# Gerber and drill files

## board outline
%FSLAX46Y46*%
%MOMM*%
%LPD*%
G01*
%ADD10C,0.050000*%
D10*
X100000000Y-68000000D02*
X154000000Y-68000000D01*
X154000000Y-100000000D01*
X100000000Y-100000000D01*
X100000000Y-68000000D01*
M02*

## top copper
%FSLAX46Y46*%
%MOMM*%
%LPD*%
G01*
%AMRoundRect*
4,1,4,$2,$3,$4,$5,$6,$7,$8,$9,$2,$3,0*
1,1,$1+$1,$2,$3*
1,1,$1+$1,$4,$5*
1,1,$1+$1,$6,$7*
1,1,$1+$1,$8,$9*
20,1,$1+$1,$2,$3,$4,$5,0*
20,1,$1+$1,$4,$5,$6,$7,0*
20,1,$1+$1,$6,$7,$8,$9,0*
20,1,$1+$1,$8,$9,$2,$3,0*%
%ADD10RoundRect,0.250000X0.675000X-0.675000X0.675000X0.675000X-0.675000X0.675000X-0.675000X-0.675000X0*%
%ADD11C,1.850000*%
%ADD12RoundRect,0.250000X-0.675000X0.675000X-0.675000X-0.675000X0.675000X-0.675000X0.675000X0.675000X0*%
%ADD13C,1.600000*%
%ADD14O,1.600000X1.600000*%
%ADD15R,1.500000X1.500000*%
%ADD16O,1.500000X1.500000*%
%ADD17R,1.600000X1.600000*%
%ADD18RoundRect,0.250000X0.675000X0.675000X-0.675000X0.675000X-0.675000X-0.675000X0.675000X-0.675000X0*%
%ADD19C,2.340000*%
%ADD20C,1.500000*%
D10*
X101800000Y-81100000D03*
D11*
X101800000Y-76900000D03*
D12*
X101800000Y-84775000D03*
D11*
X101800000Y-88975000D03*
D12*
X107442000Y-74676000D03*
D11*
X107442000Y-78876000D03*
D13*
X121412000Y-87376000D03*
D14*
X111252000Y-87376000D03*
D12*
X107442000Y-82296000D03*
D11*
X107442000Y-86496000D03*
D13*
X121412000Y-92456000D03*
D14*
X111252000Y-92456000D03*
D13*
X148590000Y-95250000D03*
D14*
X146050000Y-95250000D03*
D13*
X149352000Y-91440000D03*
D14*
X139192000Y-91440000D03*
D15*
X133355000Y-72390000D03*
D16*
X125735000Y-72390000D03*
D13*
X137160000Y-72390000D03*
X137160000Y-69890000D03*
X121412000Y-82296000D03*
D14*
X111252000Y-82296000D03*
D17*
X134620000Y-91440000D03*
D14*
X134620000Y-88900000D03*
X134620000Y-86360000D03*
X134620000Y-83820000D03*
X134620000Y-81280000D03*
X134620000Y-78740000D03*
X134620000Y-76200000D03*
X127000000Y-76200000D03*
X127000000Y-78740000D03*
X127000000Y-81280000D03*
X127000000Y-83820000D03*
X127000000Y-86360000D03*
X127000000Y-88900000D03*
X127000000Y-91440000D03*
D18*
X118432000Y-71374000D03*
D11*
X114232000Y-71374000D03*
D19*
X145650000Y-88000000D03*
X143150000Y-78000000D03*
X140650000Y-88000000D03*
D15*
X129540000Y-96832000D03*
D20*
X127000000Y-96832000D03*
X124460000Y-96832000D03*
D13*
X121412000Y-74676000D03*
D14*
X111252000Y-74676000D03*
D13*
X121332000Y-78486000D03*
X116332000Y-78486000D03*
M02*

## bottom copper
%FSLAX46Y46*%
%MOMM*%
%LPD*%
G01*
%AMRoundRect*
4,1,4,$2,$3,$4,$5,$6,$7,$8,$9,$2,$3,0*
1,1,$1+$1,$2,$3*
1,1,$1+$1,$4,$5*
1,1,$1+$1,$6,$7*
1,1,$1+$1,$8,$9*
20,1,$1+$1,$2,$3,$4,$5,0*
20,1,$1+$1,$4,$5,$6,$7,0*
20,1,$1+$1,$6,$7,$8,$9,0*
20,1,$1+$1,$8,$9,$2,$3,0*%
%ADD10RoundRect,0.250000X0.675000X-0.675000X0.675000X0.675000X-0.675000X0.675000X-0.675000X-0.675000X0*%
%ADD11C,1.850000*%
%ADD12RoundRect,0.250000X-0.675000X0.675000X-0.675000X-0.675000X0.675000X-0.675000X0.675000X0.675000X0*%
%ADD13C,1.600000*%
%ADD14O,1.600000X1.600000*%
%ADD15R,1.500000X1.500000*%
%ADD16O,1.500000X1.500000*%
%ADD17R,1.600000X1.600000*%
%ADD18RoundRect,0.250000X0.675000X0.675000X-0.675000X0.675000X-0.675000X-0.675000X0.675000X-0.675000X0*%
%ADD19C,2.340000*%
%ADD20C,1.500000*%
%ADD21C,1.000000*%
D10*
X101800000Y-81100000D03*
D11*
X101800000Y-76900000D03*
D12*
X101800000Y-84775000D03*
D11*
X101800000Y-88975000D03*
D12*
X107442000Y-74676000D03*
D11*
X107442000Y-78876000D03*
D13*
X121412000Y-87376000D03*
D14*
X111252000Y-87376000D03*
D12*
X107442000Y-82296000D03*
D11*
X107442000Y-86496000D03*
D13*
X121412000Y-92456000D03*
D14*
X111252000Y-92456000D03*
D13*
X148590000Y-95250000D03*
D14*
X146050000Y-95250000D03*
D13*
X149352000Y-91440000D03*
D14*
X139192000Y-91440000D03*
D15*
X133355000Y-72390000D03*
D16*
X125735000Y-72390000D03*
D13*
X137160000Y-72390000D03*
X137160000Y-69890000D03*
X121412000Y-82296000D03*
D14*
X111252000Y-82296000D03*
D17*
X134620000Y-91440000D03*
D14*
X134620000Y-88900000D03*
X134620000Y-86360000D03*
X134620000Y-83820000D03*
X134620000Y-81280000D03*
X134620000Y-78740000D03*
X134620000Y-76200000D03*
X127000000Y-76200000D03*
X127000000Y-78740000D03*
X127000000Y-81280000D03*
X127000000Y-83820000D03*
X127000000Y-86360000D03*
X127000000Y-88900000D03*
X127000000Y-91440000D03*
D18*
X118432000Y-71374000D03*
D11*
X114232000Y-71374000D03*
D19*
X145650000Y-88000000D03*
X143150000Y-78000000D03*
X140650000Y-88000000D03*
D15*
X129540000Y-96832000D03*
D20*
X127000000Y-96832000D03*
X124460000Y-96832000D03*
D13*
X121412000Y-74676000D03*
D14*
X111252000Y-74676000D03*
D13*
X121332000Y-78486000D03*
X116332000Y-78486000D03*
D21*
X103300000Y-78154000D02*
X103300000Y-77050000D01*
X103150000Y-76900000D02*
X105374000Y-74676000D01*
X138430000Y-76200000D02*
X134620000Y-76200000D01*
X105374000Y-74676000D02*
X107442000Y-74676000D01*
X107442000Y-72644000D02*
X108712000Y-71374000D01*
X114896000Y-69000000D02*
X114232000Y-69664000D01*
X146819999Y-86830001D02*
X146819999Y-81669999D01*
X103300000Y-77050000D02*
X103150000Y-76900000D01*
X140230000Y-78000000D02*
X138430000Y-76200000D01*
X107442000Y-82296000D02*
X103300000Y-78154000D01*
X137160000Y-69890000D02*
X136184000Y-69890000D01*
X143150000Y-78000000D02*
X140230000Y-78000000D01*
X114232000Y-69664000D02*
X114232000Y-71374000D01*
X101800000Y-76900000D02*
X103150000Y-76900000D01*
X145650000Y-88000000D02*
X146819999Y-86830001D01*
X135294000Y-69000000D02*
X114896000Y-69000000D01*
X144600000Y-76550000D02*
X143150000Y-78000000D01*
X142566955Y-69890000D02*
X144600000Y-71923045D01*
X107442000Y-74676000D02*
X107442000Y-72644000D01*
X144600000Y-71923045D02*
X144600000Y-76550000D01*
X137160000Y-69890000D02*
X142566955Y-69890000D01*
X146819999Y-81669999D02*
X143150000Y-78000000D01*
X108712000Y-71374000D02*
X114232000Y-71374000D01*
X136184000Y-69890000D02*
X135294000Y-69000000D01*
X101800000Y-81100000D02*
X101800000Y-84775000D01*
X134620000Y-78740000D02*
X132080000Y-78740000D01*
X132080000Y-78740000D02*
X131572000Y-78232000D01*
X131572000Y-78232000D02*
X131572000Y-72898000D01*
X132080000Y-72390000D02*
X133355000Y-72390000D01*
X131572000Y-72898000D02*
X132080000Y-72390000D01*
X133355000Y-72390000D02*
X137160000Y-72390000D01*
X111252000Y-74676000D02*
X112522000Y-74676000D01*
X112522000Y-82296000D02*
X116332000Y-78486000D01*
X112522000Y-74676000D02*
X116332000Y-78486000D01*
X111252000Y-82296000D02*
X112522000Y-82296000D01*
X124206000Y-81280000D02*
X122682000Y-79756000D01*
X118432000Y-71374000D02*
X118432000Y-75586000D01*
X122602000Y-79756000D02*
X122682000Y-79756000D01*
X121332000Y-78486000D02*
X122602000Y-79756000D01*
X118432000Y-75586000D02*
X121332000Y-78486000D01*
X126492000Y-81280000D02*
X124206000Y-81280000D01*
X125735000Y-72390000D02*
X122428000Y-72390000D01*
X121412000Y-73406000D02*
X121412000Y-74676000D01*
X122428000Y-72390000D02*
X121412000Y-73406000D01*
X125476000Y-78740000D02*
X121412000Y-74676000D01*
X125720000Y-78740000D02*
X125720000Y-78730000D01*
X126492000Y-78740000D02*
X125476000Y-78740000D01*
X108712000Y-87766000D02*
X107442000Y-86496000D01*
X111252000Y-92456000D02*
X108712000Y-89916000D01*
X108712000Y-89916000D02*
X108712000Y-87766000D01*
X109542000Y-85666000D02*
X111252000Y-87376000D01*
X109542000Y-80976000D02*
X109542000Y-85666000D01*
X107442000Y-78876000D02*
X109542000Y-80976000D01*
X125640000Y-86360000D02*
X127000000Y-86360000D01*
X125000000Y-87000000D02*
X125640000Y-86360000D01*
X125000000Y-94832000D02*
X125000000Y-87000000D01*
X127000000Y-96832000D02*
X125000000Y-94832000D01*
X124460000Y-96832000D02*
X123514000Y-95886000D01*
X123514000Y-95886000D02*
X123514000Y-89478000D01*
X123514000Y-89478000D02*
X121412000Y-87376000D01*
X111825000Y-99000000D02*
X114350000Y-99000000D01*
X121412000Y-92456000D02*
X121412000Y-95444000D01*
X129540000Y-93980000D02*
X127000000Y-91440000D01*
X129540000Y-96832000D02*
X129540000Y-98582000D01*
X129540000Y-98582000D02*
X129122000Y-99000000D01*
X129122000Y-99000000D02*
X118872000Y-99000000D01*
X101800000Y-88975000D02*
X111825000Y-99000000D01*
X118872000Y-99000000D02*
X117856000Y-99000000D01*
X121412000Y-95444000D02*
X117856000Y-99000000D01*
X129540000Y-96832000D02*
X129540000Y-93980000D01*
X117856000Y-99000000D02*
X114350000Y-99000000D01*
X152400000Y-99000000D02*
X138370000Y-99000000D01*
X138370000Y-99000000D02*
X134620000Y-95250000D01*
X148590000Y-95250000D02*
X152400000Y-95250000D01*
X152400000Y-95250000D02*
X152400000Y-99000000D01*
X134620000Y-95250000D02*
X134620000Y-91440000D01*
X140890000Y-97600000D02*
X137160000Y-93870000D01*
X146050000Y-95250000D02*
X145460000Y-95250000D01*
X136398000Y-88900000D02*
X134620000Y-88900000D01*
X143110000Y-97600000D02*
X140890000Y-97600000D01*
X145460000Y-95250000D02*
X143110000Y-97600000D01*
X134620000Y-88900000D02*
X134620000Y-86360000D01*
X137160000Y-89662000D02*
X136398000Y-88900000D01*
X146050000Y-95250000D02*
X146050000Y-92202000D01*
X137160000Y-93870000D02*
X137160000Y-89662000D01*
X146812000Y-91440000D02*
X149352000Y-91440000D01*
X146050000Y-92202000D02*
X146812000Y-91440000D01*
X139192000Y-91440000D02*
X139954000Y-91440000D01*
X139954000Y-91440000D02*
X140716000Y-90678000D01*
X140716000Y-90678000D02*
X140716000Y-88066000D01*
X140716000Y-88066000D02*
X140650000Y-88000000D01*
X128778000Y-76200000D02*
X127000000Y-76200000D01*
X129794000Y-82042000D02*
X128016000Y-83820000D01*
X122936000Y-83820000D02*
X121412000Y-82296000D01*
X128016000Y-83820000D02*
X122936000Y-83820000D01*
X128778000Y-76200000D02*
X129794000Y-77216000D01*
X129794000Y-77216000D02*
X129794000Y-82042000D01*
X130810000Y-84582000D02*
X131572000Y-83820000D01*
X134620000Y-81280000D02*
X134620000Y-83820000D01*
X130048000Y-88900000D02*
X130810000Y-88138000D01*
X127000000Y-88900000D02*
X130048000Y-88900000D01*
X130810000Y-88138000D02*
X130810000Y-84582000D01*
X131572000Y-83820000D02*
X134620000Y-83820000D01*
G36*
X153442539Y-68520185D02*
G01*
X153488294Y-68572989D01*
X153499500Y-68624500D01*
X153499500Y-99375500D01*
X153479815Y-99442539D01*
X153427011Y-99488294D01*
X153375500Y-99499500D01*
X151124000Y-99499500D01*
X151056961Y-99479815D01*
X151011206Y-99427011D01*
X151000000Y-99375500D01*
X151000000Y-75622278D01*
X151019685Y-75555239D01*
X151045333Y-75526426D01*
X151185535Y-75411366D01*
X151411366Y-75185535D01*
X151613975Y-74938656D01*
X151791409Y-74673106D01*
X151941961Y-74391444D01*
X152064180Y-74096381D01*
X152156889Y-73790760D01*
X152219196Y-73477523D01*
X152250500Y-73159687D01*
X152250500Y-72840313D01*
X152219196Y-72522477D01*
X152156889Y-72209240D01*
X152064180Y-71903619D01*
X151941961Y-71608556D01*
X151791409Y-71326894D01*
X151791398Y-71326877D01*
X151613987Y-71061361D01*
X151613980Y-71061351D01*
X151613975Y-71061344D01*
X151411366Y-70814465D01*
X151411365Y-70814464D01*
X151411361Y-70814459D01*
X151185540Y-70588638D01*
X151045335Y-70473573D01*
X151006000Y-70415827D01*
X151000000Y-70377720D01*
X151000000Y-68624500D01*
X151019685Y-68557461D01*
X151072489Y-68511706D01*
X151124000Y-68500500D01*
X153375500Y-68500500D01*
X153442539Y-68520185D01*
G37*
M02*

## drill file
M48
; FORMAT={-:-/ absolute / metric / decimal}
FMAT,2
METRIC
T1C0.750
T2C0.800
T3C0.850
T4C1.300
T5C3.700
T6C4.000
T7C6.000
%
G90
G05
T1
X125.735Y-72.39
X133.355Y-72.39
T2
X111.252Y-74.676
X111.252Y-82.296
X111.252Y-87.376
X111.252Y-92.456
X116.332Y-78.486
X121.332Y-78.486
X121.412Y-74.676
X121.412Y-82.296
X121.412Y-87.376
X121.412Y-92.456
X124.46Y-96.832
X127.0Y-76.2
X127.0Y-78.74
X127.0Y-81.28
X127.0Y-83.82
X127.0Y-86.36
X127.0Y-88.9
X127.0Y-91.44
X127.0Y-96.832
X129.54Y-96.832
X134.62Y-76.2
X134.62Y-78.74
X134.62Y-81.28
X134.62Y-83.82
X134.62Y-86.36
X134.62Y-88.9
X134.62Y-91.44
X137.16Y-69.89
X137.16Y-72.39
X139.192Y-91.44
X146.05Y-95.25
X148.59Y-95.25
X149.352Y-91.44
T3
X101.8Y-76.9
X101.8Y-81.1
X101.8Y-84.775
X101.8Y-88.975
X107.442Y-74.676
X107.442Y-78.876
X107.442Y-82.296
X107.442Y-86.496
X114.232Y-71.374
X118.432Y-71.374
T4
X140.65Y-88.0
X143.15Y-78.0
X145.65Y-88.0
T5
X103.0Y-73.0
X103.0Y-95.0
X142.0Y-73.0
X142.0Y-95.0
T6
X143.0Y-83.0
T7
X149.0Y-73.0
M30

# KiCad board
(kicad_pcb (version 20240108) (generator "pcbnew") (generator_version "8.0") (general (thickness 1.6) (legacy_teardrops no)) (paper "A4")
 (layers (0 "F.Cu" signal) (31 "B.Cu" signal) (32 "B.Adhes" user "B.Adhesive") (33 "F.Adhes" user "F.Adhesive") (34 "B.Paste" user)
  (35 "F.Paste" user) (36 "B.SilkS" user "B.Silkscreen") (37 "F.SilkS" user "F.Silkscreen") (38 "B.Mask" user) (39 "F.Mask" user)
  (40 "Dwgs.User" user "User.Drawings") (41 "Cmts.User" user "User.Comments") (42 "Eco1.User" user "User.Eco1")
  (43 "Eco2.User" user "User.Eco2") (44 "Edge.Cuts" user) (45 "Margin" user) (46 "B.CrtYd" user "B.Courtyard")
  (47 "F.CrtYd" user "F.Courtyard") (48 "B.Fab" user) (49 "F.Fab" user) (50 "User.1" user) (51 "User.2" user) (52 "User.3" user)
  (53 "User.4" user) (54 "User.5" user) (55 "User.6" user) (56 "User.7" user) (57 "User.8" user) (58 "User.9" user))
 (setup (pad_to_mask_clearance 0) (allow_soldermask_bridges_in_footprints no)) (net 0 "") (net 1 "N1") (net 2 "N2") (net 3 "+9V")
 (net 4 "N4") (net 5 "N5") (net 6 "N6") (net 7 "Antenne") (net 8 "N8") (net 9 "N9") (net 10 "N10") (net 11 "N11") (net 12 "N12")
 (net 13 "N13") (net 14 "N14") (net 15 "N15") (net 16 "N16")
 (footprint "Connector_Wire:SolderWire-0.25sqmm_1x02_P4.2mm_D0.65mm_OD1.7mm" (layer "F.Cu") (at 101.8 81.1 90)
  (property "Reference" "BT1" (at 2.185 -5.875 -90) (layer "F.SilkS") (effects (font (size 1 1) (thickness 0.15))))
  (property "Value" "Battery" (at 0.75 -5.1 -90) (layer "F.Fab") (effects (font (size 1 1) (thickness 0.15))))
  (pad "1" thru_hole roundrect (at 0 0 90) (size 1.85 1.85) (drill 0.85) (layers "*.Cu" "*.Mask") (remove_unused_layers no)
   (roundrect_rratio 0.135135) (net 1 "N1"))
  (pad "2" thru_hole circle (at 4.2 0 90) (size 1.85 1.85) (drill 0.85) (layers "*.Cu" "*.Mask") (remove_unused_layers no) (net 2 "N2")))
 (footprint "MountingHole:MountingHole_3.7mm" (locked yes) (layer "F.Cu") (at 142 95)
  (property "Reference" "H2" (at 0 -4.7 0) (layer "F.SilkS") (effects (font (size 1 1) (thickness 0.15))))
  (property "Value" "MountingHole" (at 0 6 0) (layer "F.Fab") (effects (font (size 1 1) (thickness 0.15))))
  (pad "" np_thru_hole circle (at 0 0) (size 3.7 3.7) (drill 3.7) (layers "*.Cu" "*.Mask")))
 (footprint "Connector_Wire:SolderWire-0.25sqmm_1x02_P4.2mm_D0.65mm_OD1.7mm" (layer "F.Cu") (at 101.8 84.775 -90)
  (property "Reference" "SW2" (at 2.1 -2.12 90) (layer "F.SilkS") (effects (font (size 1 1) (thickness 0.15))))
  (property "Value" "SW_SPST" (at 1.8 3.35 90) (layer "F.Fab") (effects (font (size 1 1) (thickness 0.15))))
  (pad "1" thru_hole roundrect (at 0 0 270) (size 1.85 1.85) (drill 0.85) (layers "*.Cu" "*.Mask") (remove_unused_layers no)
   (roundrect_rratio 0.135135) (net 1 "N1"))
  (pad "2" thru_hole circle (at 4.2 0 270) (size 1.85 1.85) (drill 0.85) (layers "*.Cu" "*.Mask") (remove_unused_layers no) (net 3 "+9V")))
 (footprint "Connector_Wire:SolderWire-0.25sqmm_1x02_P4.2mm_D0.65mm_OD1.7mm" (layer "F.Cu") (at 107.442 74.676 -90)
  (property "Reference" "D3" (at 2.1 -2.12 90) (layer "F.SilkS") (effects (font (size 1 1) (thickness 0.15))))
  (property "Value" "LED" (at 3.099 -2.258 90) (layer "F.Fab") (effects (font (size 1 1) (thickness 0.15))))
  (pad "1" thru_hole roundrect (at 0 0 270) (size 1.85 1.85) (drill 0.85) (layers "*.Cu" "*.Mask") (remove_unused_layers no)
   (roundrect_rratio 0.135135) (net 2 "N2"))
  (pad "2" thru_hole circle (at 4.2 0 270) (size 1.85 1.85) (drill 0.85) (layers "*.Cu" "*.Mask") (remove_unused_layers no) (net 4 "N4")))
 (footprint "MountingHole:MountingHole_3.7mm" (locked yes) (layer "F.Cu") (at 142 73)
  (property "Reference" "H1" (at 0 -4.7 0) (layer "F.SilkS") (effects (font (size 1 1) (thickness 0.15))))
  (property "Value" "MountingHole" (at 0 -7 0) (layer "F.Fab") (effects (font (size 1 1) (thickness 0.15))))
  (pad "" np_thru_hole circle (at 0 0) (size 3.7 3.7) (drill 3.7) (layers "*.Cu" "*.Mask")))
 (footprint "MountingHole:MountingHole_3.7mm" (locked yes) (layer "F.Cu") (at 103 73)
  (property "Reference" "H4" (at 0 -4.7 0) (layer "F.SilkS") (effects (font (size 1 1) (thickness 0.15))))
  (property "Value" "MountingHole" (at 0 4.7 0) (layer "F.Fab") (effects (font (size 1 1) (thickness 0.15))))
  (pad "" np_thru_hole circle (at 0 0) (size 3.7 3.7) (drill 3.7) (layers "*.Cu" "*.Mask")))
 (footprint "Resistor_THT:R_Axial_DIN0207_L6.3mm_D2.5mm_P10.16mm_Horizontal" (layer "F.Cu") (at 121.412 87.376 180)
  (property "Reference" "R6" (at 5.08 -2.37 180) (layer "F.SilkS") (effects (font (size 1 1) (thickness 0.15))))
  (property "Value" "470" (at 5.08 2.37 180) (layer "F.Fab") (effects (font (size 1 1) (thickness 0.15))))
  (pad "1" thru_hole circle (at 0 0 180) (size 1.6 1.6) (drill 0.8) (layers "*.Cu" "*.Mask") (remove_unused_layers no) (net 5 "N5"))
  (pad "2" thru_hole oval (at 10.16 0 180) (size 1.6 1.6) (drill 0.8) (layers "*.Cu" "*.Mask") (remove_unused_layers no) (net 4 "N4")))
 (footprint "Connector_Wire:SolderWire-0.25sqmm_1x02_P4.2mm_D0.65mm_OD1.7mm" (layer "F.Cu") (at 107.442 82.296 -90)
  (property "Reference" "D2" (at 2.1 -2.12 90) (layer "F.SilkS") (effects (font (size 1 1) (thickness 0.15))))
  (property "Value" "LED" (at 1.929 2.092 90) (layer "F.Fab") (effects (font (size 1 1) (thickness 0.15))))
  (pad "1" thru_hole roundrect (at 0 0 270) (size 1.85 1.85) (drill 0.85) (layers "*.Cu" "*.Mask") (remove_unused_layers no)
   (roundrect_rratio 0.135135) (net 2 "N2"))
  (pad "2" thru_hole circle (at 4.2 0 270) (size 1.85 1.85) (drill 0.85) (layers "*.Cu" "*.Mask") (remove_unused_layers no) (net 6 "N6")))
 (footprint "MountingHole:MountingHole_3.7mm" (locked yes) (layer "F.Cu") (at 103 95)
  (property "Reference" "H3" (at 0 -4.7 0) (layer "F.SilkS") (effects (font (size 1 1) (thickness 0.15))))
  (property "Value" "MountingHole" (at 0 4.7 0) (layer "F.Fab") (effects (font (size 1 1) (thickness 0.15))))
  (pad "" np_thru_hole circle (at 0 0) (size 3.7 3.7) (drill 3.7) (layers "*.Cu" "*.Mask")))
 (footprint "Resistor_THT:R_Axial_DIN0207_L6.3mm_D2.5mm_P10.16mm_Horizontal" (layer "F.Cu") (at 121.412 92.456 180)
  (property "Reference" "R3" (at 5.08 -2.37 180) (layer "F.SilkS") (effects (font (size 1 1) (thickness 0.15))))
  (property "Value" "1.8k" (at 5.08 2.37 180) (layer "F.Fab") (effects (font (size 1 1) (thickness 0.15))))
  (pad "1" thru_hole circle (at 0 0 180) (size 1.6 1.6) (drill 0.8) (layers "*.Cu" "*.Mask") (remove_unused_layers no) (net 3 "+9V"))
  (pad "2" thru_hole oval (at 10.16 0 180) (size 1.6 1.6) (drill 0.8) (layers "*.Cu" "*.Mask") (remove_unused_layers no) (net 6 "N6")))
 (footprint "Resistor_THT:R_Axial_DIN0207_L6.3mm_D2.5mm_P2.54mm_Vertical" (layer "F.Cu") (at 148.59 95.25 180)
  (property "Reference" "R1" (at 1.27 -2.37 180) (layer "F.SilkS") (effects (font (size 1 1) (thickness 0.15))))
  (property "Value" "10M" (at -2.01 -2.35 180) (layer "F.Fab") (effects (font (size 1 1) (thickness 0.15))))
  (pad "1" thru_hole circle (at 0 0 180) (size 1.6 1.6) (drill 0.8) (layers "*.Cu" "*.Mask") (remove_unused_layers no) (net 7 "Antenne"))
  (pad "2" thru_hole oval (at 2.54 0 180) (size 1.6 1.6) (drill 0.8) (layers "*.Cu" "*.Mask") (remove_unused_layers no) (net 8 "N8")))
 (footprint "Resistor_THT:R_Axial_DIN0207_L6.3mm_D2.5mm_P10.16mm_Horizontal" (layer "F.Cu") (at 149.352 91.44 180)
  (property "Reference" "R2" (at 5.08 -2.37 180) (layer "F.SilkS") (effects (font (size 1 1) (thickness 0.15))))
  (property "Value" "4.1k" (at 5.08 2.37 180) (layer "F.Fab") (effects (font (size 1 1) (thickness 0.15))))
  (pad "1" thru_hole circle (at 0 0 180) (size 1.6 1.6) (drill 0.8) (layers "*.Cu" "*.Mask") (remove_unused_layers no) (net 8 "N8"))
  (pad "2" thru_hole oval (at 10.16 0 180) (size 1.6 1.6) (drill 0.8) (layers "*.Cu" "*.Mask") (remove_unused_layers no) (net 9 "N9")))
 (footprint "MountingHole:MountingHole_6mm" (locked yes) (layer "F.Cu") (at 149 73)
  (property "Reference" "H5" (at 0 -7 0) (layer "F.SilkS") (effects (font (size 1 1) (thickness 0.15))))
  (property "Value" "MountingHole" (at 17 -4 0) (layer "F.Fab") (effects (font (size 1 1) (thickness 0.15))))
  (pad "" np_thru_hole circle (at 0 0) (size 6 6) (drill 6) (layers "*.Cu" "*.Mask")))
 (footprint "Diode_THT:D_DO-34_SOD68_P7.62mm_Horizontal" (layer "F.Cu") (at 133.355 72.39 180)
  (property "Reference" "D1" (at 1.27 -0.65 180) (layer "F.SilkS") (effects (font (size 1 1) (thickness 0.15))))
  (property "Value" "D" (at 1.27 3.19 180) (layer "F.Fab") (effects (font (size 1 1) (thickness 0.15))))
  (pad "1" thru_hole rect (at 0 0 180) (size 1.5 1.5) (drill 0.75) (layers "*.Cu" "*.Mask") (remove_unused_layers no) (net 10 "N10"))
  (pad "2" thru_hole oval (at 7.62 0 180) (size 1.5 1.5) (drill 0.75) (layers "*.Cu" "*.Mask") (remove_unused_layers no) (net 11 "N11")))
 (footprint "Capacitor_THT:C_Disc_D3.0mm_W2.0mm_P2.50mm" (layer "F.Cu") (at 137.16 72.39 90)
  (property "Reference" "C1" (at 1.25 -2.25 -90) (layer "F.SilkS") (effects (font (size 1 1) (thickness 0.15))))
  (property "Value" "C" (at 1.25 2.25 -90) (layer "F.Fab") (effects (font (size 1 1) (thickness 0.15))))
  (pad "1" thru_hole circle (at 0 0 90) (size 1.6 1.6) (drill 0.8) (layers "*.Cu" "*.Mask") (remove_unused_layers no) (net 10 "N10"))
  (pad "2" thru_hole circle (at 2.5 0 90) (size 1.6 1.6) (drill 0.8) (layers "*.Cu" "*.Mask") (remove_unused_layers no) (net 2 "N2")))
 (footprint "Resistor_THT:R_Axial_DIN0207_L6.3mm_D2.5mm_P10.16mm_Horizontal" (layer "F.Cu") (at 121.412 82.296 180)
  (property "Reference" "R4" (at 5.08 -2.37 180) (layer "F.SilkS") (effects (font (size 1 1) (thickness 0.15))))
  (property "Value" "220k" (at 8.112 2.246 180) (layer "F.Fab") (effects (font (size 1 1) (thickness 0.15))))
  (pad "1" thru_hole circle (at 0 0 180) (size 1.6 1.6) (drill 0.8) (layers "*.Cu" "*.Mask") (remove_unused_layers no) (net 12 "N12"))
  (pad "2" thru_hole oval (at 10.16 0 180) (size 1.6 1.6) (drill 0.8) (layers "*.Cu" "*.Mask") (remove_unused_layers no) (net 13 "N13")))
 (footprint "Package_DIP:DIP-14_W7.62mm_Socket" (layer "F.Cu") (at 134.62 91.44 180)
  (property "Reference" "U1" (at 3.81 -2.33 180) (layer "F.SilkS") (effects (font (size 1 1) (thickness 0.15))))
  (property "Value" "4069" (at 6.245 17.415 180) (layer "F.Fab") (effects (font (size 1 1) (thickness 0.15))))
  (pad "1" thru_hole rect (at 0 0 180) (size 1.6 1.6) (drill 0.8) (layers "*.Cu" "*.Mask") (remove_unused_layers no) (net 7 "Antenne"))
  (pad "2" thru_hole oval (at 0 2.54 180) (size 1.6 1.6) (drill 0.8) (layers "*.Cu" "*.Mask") (remove_unused_layers no) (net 8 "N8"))
  (pad "3" thru_hole oval (at 0 5.08 180) (size 1.6 1.6) (drill 0.8) (layers "*.Cu" "*.Mask") (remove_unused_layers no) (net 8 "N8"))
  (pad "4" thru_hole oval (at 0 7.62 180) (size 1.6 1.6) (drill 0.8) (layers "*.Cu" "*.Mask") (remove_unused_layers no) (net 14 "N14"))
  (pad "5" thru_hole oval (at 0 10.16 180) (size 1.6 1.6) (drill 0.8) (layers "*.Cu" "*.Mask") (remove_unused_layers no) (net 14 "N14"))
  (pad "6" thru_hole oval (at 0 12.7 180) (size 1.6 1.6) (drill 0.8) (layers "*.Cu" "*.Mask") (remove_unused_layers no) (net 10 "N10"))
  (pad "7" thru_hole oval (at 0 15.24 180) (size 1.6 1.6) (drill 0.8) (layers "*.Cu" "*.Mask") (remove_unused_layers no) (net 2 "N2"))
  (pad "8" thru_hole oval (at 7.62 15.24 180) (size 1.6 1.6) (drill 0.8) (layers "*.Cu" "*.Mask") (remove_unused_layers no) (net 12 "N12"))
  (pad "9" thru_hole oval (at 7.62 12.7 180) (size 1.6 1.6) (drill 0.8) (layers "*.Cu" "*.Mask") (remove_unused_layers no) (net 11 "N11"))
  (pad "10" thru_hole oval (at 7.62 10.16 180) (size 1.6 1.6) (drill 0.8) (layers "*.Cu" "*.Mask") (remove_unused_layers no) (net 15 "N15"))
  (pad "11" thru_hole oval (at 7.62 7.62 180) (size 1.6 1.6) (drill 0.8) (layers "*.Cu" "*.Mask") (remove_unused_layers no) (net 12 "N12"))
  (pad "12" thru_hole oval (at 7.62 5.08 180) (size 1.6 1.6) (drill 0.8) (layers "*.Cu" "*.Mask") (remove_unused_layers no) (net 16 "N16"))
  (pad "13" thru_hole oval (at 7.62 2.54 180) (size 1.6 1.6) (drill 0.8) (layers "*.Cu" "*.Mask") (remove_unused_layers no) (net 14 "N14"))
  (pad "14" thru_hole oval (at 7.62 0 180) (size 1.6 1.6) (drill 0.8) (layers "*.Cu" "*.Mask") (remove_unused_layers no) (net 3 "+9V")))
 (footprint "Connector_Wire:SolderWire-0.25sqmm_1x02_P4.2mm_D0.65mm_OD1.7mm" (layer "F.Cu") (at 118.432 71.374 180)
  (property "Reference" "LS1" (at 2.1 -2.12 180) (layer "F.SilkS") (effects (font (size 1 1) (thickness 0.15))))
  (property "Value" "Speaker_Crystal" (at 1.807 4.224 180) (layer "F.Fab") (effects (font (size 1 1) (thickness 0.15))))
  (pad "1" thru_hole roundrect (at 0 0 180) (size 1.85 1.85) (drill 0.85) (layers "*.Cu" "*.Mask") (remove_unused_layers no)
   (roundrect_rratio 0.135135) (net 15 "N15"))
  (pad "2" thru_hole circle (at 4.2 0 180) (size 1.85 1.85) (drill 0.85) (layers "*.Cu" "*.Mask") (remove_unused_layers no) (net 2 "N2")))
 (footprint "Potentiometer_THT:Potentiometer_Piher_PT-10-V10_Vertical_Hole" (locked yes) (layer "F.Cu") (at 145.65 88 90)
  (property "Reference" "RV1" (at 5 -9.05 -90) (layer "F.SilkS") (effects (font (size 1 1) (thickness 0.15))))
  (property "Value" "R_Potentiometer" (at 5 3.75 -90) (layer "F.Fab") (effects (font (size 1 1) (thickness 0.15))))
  (pad "" np_thru_hole circle (at 5 -2.65 90) (size 4 4) (drill 4) (layers "*.Cu" "*.Mask"))
  (pad "1" thru_hole circle (at 0 0 90) (size 2.34 2.34) (drill 1.3) (layers "*.Cu" "*.Mask") (remove_unused_layers no) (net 2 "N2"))
  (pad "2" thru_hole circle (at 10 -2.5 90) (size 2.34 2.34) (drill 1.3) (layers "*.Cu" "*.Mask") (remove_unused_layers no) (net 2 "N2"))
  (pad "3" thru_hole circle (at 0 -5 90) (size 2.34 2.34) (drill 1.3) (layers "*.Cu" "*.Mask") (remove_unused_layers no) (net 9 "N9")))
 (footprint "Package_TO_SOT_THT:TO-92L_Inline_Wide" (layer "F.Cu") (at 129.54 96.832 180)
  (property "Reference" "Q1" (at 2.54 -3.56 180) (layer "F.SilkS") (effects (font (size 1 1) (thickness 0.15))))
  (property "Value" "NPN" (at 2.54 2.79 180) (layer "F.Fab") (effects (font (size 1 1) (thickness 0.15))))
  (pad "1" thru_hole rect (at 0 0 180) (size 1.5 1.5) (drill 0.8) (layers "*.Cu" "*.Mask") (remove_unused_layers no) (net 3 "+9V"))
  (pad "2" thru_hole circle (at 2.54 0 180) (size 1.5 1.5) (drill 0.8) (layers "*.Cu" "*.Mask") (remove_unused_layers no) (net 16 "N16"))
  (pad "3" thru_hole circle (at 5.08 0 180) (size 1.5 1.5) (drill 0.8) (layers "*.Cu" "*.Mask") (remove_unused_layers no) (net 5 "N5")))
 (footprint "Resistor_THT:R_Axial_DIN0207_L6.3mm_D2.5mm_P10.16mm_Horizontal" (layer "F.Cu") (at 121.412 74.676 180)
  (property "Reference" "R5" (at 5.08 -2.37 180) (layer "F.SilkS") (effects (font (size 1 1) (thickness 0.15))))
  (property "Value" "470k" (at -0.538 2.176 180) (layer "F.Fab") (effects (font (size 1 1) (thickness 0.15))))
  (pad "1" thru_hole circle (at 0 0 180) (size 1.6 1.6) (drill 0.8) (layers "*.Cu" "*.Mask") (remove_unused_layers no) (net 11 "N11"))
  (pad "2" thru_hole oval (at 10.16 0 180) (size 1.6 1.6) (drill 0.8) (layers "*.Cu" "*.Mask") (remove_unused_layers no) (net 13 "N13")))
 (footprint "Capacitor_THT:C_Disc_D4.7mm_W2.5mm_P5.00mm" (layer "F.Cu") (at 121.332 78.486 180)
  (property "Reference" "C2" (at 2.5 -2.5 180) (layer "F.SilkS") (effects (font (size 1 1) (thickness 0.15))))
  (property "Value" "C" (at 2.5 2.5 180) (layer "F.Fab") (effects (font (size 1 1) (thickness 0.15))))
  (pad "1" thru_hole circle (at 0 0 180) (size 1.6 1.6) (drill 0.8) (layers "*.Cu" "*.Mask") (remove_unused_layers no) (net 15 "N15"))
  (pad "2" thru_hole circle (at 5 0 180) (size 1.6 1.6) (drill 0.8) (layers "*.Cu" "*.Mask") (remove_unused_layers no) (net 13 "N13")))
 (gr_rect (start 100 68) (end 154 100) (locked yes) (stroke (width 0.05) (type default)) (fill none) (layer "Edge.Cuts"))
 (segment (start 103.3 78.154) (end 103.3 77.05) (width 1) (layer "B.Cu") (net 2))
 (segment (start 103.15 76.9) (end 105.374 74.676) (width 1) (layer "B.Cu") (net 2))
 (segment (start 138.43 76.2) (end 134.62 76.2) (width 1) (layer "B.Cu") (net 2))
 (segment (start 105.374 74.676) (end 107.442 74.676) (width 1) (layer "B.Cu") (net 2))
 (segment (start 107.442 72.644) (end 108.712 71.374) (width 1) (layer "B.Cu") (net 2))
 (segment (start 114.896 69) (end 114.232 69.664) (width 1) (layer "B.Cu") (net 2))
 (segment (start 146.819999 86.830001) (end 146.819999 81.669999) (width 1) (layer "B.Cu") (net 2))
 (segment (start 103.3 77.05) (end 103.15 76.9) (width 1) (layer "B.Cu") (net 2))
 (segment (start 140.23 78) (end 138.43 76.2) (width 1) (layer "B.Cu") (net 2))
 (segment (start 107.442 82.296) (end 103.3 78.154) (width 1) (layer "B.Cu") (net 2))
 (segment (start 137.16 69.89) (end 136.184 69.89) (width 1) (layer "B.Cu") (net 2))
 (segment (start 143.15 78) (end 140.23 78) (width 1) (layer "B.Cu") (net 2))
 (segment (start 114.232 69.664) (end 114.232 71.374) (width 1) (layer "B.Cu") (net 2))
 (segment (start 101.8 76.9) (end 103.15 76.9) (width 1) (layer "B.Cu") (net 2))
 (segment (start 145.65 88) (end 146.819999 86.830001) (width 1) (layer "B.Cu") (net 2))
 (segment (start 135.294 69) (end 114.896 69) (width 1) (layer "B.Cu") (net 2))
 (segment (start 144.6 76.55) (end 143.15 78) (width 1) (layer "B.Cu") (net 2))
 (segment (start 142.566955 69.89) (end 144.6 71.923045) (width 1) (layer "B.Cu") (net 2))
 (segment (start 107.442 74.676) (end 107.442 72.644) (width 1) (layer "B.Cu") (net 2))
 (segment (start 144.6 71.923045) (end 144.6 76.55) (width 1) (layer "B.Cu") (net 2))
 (segment (start 137.16 69.89) (end 142.566955 69.89) (width 1) (layer "B.Cu") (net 2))
 (segment (start 146.819999 81.669999) (end 143.15 78) (width 1) (layer "B.Cu") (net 2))
 (segment (start 108.712 71.374) (end 114.232 71.374) (width 1) (layer "B.Cu") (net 2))
 (segment (start 136.184 69.89) (end 135.294 69) (width 1) (layer "B.Cu") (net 2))
 (segment (start 101.8 81.1) (end 101.8 84.775) (width 1) (layer "B.Cu") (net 1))
 (segment (start 134.62 78.74) (end 132.08 78.74) (width 1) (layer "B.Cu") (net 10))
 (segment (start 132.08 78.74) (end 131.572 78.232) (width 1) (layer "B.Cu") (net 10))
 (segment (start 131.572 78.232) (end 131.572 72.898) (width 1) (layer "B.Cu") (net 10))
 (segment (start 132.08 72.39) (end 133.355 72.39) (width 1) (layer "B.Cu") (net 10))
 (segment (start 131.572 72.898) (end 132.08 72.39) (width 1) (layer "B.Cu") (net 10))
 (segment (start 133.355 72.39) (end 137.16 72.39) (width 1) (layer "B.Cu") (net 10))
 (segment (start 111.252 74.676) (end 112.522 74.676) (width 1) (layer "B.Cu") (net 13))
 (segment (start 112.522 82.296) (end 116.332 78.486) (width 1) (layer "B.Cu") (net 13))
 (segment (start 112.522 74.676) (end 116.332 78.486) (width 1) (layer "B.Cu") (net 13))
 (segment (start 111.252 82.296) (end 112.522 82.296) (width 1) (layer "B.Cu") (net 13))
 (segment (start 124.206 81.28) (end 122.682 79.756) (width 1) (layer "B.Cu") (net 15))
 (segment (start 118.432 71.374) (end 118.432 75.586) (width 1) (layer "B.Cu") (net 15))
 (segment (start 122.602 79.756) (end 122.682 79.756) (width 1) (layer "B.Cu") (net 15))
 (segment (start 121.332 78.486) (end 122.602 79.756) (width 1) (layer "B.Cu") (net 15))
 (segment (start 118.432 75.586) (end 121.332 78.486) (width 1) (layer "B.Cu") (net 15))
 (segment (start 126.492 81.28) (end 124.206 81.28) (width 1) (layer "B.Cu") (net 15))
 (segment (start 125.735 72.39) (end 122.428 72.39) (width 1) (layer "B.Cu") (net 11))
 (segment (start 121.412 73.406) (end 121.412 74.676) (width 1) (layer "B.Cu") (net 11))
 (segment (start 122.428 72.39) (end 121.412 73.406) (width 1) (layer "B.Cu") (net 11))
 (segment (start 125.476 78.74) (end 121.412 74.676) (width 1) (layer "B.Cu") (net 11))
 (segment (start 125.72 78.74) (end 125.72 78.73) (width 1) (layer "B.Cu") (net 11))
 (segment (start 126.492 78.74) (end 125.476 78.74) (width 1) (layer "B.Cu") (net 11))
 (segment (start 108.712 87.766) (end 107.442 86.496) (width 1) (layer "B.Cu") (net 6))
 (segment (start 111.252 92.456) (end 108.712 89.916) (width 1) (layer "B.Cu") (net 6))
 (segment (start 108.712 89.916) (end 108.712 87.766) (width 1) (layer "B.Cu") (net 6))
 (segment (start 109.542 85.666) (end 111.252 87.376) (width 1) (layer "B.Cu") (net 4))
 (segment (start 109.542 80.976) (end 109.542 85.666) (width 1) (layer "B.Cu") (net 4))
 (segment (start 107.442 78.876) (end 109.542 80.976) (width 1) (layer "B.Cu") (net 4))
 (segment (start 125.64 86.36) (end 127 86.36) (width 1) (layer "B.Cu") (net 16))
 (segment (start 125 87) (end 125.64 86.36) (width 1) (layer "B.Cu") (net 16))
 (segment (start 125 94.832) (end 125 87) (width 1) (layer "B.Cu") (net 16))
 (segment (start 127 96.832) (end 125 94.832) (width 1) (layer "B.Cu") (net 16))
 (segment (start 124.46 96.832) (end 123.514 95.886) (width 1) (layer "B.Cu") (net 5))
 (segment (start 123.514 95.886) (end 123.514 89.478) (width 1) (layer "B.Cu") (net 5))
 (segment (start 123.514 89.478) (end 121.412 87.376) (width 1) (layer "B.Cu") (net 5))
 (segment (start 111.825 99) (end 114.35 99) (width 1) (layer "B.Cu") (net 3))
 (segment (start 121.412 92.456) (end 121.412 95.444) (width 1) (layer "B.Cu") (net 3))
 (segment (start 129.54 93.98) (end 127 91.44) (width 1) (layer "B.Cu") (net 3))
 (segment (start 129.54 96.832) (end 129.54 98.582) (width 1) (layer "B.Cu") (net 3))
 (segment (start 129.54 98.582) (end 129.122 99) (width 1) (layer "B.Cu") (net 3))
 (segment (start 129.122 99) (end 118.872 99) (width 1) (layer "B.Cu") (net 3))
 (segment (start 101.8 88.975) (end 111.825 99) (width 1) (layer "B.Cu") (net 3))
 (segment (start 118.872 99) (end 117.856 99) (width 1) (layer "B.Cu") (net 3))
 (segment (start 121.412 95.444) (end 117.856 99) (width 1) (layer "B.Cu") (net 3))
 (segment (start 129.54 96.832) (end 129.54 93.98) (width 1) (layer "B.Cu") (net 3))
 (segment (start 117.856 99) (end 114.35 99) (width 1) (layer "B.Cu") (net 3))
 (segment (start 152.4 99) (end 138.37 99) (width 1) (layer "B.Cu") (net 7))
 (segment (start 138.37 99) (end 134.62 95.25) (width 1) (layer "B.Cu") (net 7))
 (segment (start 148.59 95.25) (end 152.4 95.25) (width 1) (layer "B.Cu") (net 7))
 (segment (start 152.4 95.25) (end 152.4 99) (width 1) (layer "B.Cu") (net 7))
 (segment (start 134.62 95.25) (end 134.62 91.44) (width 1) (layer "B.Cu") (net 7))
 (segment (start 140.89 97.6) (end 137.16 93.87) (width 1) (layer "B.Cu") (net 8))
 (segment (start 146.05 95.25) (end 145.46 95.25) (width 1) (layer "B.Cu") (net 8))
 (segment (start 136.398 88.9) (end 134.62 88.9) (width 1) (layer "B.Cu") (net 8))
 (segment (start 143.11 97.6) (end 140.89 97.6) (width 1) (layer "B.Cu") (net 8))
 (segment (start 145.46 95.25) (end 143.11 97.6) (width 1) (layer "B.Cu") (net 8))
 (segment (start 134.62 88.9) (end 134.62 86.36) (width 1) (layer "B.Cu") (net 8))
 (segment (start 137.16 89.662) (end 136.398 88.9) (width 1) (layer "B.Cu") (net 8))
 (segment (start 146.05 95.25) (end 146.05 92.202) (width 1) (layer "B.Cu") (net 8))
 (segment (start 137.16 93.87) (end 137.16 89.662) (width 1) (layer "B.Cu") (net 8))
 (segment (start 146.812 91.44) (end 149.352 91.44) (width 1) (layer "B.Cu") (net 8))
 (segment (start 146.05 92.202) (end 146.812 91.44) (width 1) (layer "B.Cu") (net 8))
 (segment (start 139.192 91.44) (end 139.954 91.44) (width 1) (layer "B.Cu") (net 9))
 (segment (start 139.954 91.44) (end 140.716 90.678) (width 1) (layer "B.Cu") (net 9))
 (segment (start 140.716 90.678) (end 140.716 88.066) (width 1) (layer "B.Cu") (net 9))
 (segment (start 140.716 88.066) (end 140.65 88) (width 1) (layer "B.Cu") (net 9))
 (segment (start 128.778 76.2) (end 127 76.2) (width 1) (layer "B.Cu") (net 12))
 (segment (start 129.794 82.042) (end 128.016 83.82) (width 1) (layer "B.Cu") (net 12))
 (segment (start 122.936 83.82) (end 121.412 82.296) (width 1) (layer "B.Cu") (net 12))
 (segment (start 128.016 83.82) (end 122.936 83.82) (width 1) (layer "B.Cu") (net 12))
 (segment (start 128.778 76.2) (end 129.794 77.216) (width 1) (layer "B.Cu") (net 12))
 (segment (start 129.794 77.216) (end 129.794 82.042) (width 1) (layer "B.Cu") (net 12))
 (segment (start 130.81 84.582) (end 131.572 83.82) (width 1) (layer "B.Cu") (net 14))
 (segment (start 134.62 81.28) (end 134.62 83.82) (width 1) (layer "B.Cu") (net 14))
 (segment (start 130.048 88.9) (end 130.81 88.138) (width 1) (layer "B.Cu") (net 14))
 (segment (start 127 88.9) (end 130.048 88.9) (width 1) (layer "B.Cu") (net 14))
 (segment (start 130.81 88.138) (end 130.81 84.582) (width 1) (layer "B.Cu") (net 14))
 (segment (start 131.572 83.82) (end 134.62 83.82) (width 1) (layer "B.Cu") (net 14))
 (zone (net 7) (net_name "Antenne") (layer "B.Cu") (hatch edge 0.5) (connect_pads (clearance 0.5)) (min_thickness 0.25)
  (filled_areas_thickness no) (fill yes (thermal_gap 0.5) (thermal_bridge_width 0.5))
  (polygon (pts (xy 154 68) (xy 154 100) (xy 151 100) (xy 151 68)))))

